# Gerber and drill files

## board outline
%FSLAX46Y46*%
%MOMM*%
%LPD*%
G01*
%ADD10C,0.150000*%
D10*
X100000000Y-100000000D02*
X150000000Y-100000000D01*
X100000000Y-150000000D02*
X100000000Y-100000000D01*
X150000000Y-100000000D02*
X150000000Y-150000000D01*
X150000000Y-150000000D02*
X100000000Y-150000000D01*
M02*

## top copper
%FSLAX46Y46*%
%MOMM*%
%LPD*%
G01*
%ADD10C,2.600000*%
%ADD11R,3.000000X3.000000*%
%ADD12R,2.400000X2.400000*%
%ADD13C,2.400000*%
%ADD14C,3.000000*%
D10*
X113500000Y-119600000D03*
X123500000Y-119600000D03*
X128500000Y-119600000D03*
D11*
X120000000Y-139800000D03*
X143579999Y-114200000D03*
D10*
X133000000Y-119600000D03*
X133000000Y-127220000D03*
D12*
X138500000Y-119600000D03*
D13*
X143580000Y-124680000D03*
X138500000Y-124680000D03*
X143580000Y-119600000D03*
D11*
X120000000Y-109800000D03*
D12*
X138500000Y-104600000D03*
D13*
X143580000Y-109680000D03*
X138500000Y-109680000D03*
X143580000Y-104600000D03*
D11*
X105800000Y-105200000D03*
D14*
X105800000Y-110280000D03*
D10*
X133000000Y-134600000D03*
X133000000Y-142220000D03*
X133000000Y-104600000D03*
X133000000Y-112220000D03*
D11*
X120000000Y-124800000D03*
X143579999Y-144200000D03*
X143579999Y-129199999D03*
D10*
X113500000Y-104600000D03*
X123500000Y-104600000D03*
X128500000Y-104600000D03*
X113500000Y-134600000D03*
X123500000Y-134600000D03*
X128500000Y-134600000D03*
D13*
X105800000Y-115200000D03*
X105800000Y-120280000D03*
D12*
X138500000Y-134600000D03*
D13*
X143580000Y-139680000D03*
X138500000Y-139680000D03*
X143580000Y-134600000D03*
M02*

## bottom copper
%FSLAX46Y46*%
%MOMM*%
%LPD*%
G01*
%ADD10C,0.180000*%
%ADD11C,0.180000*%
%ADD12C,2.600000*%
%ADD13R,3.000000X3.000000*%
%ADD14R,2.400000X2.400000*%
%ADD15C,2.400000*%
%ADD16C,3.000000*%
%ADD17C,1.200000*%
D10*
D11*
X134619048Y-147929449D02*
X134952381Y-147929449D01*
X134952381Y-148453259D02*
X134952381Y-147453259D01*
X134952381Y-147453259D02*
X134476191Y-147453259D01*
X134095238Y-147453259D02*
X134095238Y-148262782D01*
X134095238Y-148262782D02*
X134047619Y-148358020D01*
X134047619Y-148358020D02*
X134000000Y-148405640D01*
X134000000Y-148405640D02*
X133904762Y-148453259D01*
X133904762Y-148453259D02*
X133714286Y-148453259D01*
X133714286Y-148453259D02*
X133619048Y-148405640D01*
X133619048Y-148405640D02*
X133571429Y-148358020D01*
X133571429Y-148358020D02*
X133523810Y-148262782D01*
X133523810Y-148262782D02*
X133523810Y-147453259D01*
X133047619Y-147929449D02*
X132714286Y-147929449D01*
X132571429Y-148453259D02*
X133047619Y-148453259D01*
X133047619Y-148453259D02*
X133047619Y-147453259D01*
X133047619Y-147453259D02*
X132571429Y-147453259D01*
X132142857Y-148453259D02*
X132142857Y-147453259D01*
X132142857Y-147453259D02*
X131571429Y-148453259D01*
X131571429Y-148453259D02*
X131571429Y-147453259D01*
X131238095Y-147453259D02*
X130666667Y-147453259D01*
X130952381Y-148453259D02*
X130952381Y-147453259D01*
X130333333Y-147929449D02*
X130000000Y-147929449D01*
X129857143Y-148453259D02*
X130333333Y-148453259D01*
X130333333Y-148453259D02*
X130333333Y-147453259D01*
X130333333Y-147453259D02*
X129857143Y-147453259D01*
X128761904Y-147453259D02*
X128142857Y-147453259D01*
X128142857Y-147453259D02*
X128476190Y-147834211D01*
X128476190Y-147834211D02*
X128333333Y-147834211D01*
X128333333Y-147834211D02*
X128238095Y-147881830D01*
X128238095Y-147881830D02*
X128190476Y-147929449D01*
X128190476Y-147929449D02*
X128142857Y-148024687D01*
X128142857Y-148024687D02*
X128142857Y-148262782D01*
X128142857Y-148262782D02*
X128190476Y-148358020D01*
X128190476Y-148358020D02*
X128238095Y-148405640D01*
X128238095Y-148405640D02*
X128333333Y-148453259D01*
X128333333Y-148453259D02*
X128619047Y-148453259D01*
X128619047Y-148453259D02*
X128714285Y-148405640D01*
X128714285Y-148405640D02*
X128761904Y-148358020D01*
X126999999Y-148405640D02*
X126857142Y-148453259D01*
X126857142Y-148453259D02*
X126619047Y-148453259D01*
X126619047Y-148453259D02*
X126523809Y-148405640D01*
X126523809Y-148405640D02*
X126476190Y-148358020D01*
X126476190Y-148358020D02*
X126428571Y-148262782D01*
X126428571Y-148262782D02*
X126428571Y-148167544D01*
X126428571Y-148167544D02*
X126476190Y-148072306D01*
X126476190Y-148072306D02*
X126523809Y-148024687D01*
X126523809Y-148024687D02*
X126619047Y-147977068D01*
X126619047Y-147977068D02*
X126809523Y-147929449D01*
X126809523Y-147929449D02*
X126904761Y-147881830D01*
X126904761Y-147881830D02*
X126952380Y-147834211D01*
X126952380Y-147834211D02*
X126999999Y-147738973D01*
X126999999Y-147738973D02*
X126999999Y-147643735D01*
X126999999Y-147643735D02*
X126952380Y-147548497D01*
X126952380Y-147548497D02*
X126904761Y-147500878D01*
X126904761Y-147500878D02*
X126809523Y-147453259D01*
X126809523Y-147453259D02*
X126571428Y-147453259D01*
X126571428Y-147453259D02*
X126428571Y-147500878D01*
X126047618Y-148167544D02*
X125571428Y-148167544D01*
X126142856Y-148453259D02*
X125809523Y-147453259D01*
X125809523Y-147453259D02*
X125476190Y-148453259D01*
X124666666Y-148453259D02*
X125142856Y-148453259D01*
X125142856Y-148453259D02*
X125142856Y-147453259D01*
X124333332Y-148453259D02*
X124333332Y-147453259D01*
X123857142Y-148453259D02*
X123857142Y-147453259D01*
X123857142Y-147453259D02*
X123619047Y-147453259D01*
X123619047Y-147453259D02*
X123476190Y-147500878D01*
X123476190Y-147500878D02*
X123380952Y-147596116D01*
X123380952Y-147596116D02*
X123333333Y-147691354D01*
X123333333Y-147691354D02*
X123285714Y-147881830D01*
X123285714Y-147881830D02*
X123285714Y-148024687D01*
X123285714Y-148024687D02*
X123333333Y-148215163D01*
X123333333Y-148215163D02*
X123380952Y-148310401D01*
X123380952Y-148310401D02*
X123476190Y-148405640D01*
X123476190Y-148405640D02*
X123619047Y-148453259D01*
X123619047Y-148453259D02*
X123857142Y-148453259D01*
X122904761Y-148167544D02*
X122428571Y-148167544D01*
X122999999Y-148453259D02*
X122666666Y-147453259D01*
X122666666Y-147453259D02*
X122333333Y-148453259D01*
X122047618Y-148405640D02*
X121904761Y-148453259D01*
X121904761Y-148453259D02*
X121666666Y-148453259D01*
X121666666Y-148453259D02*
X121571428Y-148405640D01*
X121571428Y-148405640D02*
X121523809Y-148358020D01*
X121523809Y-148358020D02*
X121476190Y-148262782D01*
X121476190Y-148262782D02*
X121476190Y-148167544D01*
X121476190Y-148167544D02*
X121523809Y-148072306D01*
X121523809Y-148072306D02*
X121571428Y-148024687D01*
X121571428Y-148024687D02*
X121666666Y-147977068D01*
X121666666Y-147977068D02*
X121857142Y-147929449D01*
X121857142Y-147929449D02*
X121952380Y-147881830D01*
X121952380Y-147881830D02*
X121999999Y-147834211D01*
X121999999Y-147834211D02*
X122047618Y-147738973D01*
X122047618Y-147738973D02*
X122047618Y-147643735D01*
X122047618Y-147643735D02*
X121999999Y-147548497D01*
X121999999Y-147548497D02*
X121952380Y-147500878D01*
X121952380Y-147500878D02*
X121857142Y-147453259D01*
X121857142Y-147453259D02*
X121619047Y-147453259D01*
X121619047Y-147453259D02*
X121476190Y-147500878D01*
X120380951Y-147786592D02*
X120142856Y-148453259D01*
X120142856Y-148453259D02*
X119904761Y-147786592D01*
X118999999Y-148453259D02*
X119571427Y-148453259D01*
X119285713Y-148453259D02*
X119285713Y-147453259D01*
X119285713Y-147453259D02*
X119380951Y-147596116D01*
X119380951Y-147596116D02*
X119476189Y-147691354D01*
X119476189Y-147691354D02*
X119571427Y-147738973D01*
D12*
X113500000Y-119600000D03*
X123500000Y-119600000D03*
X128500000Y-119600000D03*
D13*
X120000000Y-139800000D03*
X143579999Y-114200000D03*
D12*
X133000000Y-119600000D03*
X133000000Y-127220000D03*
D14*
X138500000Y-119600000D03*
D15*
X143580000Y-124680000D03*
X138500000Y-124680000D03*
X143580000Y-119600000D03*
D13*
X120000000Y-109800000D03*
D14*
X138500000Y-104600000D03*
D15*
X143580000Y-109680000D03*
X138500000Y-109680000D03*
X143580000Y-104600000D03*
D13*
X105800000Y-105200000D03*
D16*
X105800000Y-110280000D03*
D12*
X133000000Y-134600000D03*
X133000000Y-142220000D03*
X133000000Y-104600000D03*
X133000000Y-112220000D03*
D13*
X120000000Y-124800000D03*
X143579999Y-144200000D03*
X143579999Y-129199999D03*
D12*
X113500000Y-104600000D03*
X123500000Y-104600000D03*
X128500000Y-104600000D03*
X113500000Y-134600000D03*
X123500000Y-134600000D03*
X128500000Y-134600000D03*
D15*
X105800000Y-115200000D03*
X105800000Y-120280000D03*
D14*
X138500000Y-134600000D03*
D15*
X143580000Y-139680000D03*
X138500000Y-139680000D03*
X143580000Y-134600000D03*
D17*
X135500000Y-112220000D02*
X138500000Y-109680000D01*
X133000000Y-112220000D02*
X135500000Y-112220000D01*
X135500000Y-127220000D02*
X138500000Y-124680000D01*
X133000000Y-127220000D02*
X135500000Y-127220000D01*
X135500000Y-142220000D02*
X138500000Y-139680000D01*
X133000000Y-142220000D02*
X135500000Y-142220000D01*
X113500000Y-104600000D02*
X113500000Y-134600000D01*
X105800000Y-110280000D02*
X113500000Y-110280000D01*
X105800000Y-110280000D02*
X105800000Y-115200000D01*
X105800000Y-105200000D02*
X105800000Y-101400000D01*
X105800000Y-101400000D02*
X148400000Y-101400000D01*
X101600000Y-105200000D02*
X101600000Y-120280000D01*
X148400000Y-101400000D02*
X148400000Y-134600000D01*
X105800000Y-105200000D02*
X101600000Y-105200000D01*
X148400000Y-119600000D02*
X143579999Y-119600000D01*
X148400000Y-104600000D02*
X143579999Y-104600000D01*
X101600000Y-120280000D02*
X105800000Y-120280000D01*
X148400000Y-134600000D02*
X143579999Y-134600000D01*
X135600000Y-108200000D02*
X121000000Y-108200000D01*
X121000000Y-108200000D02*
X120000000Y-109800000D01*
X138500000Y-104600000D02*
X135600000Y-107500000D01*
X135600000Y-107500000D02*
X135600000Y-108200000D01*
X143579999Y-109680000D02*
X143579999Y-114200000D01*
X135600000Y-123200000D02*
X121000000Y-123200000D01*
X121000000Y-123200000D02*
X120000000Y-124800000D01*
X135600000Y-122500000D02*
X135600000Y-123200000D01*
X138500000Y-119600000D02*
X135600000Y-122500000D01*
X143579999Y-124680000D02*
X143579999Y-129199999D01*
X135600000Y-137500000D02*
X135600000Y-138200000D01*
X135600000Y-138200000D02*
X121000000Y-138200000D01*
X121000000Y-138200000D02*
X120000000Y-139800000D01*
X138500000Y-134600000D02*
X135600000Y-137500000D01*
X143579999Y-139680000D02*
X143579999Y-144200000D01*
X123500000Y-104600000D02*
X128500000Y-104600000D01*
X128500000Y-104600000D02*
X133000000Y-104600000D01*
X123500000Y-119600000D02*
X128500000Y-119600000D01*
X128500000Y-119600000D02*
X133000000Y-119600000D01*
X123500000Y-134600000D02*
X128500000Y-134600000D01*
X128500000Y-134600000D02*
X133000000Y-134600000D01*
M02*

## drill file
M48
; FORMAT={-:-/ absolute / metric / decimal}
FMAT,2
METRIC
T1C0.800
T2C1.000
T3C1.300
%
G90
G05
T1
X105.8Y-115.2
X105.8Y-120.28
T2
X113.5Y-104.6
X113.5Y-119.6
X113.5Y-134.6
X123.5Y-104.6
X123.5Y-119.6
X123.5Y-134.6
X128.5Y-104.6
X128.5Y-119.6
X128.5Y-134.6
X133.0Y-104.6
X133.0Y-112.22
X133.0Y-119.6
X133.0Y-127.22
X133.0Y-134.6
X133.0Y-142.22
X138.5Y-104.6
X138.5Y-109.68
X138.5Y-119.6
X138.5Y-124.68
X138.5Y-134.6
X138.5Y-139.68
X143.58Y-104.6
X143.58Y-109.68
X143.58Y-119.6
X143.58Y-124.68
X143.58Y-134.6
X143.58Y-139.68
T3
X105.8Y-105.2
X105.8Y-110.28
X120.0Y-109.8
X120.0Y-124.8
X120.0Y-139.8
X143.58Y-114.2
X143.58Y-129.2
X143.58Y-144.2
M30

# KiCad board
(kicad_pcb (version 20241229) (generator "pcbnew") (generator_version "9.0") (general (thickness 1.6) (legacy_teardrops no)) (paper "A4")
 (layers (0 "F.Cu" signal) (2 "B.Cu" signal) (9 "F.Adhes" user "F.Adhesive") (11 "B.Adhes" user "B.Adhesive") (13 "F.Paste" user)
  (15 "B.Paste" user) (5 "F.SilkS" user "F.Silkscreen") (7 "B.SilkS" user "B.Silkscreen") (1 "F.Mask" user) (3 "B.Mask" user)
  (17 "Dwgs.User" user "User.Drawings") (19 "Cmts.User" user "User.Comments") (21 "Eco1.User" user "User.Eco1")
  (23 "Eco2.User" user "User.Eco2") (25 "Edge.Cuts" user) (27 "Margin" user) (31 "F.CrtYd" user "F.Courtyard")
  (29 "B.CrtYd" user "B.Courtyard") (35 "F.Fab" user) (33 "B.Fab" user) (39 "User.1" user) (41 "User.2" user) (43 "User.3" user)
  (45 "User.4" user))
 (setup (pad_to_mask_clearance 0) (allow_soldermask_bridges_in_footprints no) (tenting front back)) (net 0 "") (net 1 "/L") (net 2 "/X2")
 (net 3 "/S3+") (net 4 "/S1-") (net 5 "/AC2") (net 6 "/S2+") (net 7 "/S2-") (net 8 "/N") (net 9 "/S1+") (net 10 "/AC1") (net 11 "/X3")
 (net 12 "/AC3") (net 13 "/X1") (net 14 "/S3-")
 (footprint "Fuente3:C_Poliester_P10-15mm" (layer "F.Cu") (at 113.5 119.6)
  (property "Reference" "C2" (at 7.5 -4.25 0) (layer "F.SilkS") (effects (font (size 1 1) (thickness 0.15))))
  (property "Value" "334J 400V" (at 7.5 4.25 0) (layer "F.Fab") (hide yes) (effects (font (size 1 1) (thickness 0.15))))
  (pad "1" thru_hole circle (at 0 0) (size 2.6 2.6) (drill 1) (layers "B.Cu" "B.Mask") (remove_unused_layers no) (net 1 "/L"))
  (pad "2" thru_hole circle (at 10 0) (size 2.6 2.6) (drill 1) (layers "B.Cu" "B.Mask") (remove_unused_layers no) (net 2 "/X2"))
  (pad "2" thru_hole circle (at 15 0) (size 2.6 2.6) (drill 1) (layers "B.Cu" "B.Mask") (remove_unused_layers no) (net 2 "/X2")))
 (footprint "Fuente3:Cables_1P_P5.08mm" (layer "F.Cu") (at 120 139.8)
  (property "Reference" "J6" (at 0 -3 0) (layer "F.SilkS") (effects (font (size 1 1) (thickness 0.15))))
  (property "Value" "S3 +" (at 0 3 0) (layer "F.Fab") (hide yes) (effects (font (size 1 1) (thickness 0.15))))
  (pad "1" thru_hole rect (at 0 0) (size 3 3) (drill 1.3) (layers "B.Cu" "B.Mask") (remove_unused_layers no) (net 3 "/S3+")))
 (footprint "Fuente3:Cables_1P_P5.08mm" (layer "F.Cu") (at 143.579999 114.2)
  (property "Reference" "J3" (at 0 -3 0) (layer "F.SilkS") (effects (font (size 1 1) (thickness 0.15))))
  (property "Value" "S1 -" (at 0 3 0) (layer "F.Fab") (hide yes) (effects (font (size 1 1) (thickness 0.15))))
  (pad "1" thru_hole rect (at 0 0) (size 3 3) (drill 1.3) (layers "B.Cu" "B.Mask") (remove_unused_layers no) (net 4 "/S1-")))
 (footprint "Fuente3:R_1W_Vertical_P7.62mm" (layer "F.Cu") (at 133 119.6 -90)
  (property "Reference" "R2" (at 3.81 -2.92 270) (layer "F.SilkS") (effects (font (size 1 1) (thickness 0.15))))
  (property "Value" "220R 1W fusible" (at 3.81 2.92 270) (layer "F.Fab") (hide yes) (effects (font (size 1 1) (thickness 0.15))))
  (pad "1" thru_hole circle (at 0 0 270) (size 2.6 2.6) (drill 1) (layers "B.Cu" "B.Mask") (remove_unused_layers no) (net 2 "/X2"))
  (pad "2" thru_hole circle (at 7.62 0 270) (size 2.6 2.6) (drill 1) (layers "B.Cu" "B.Mask") (remove_unused_layers no) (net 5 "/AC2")))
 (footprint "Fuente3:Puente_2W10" (layer "F.Cu") (at 138.5 119.6)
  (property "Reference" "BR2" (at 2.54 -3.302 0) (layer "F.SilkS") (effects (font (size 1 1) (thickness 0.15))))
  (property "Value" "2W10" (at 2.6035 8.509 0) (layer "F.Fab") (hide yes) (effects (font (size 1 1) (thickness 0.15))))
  (pad "1" thru_hole rect (at 0 0) (size 2.4 2.4) (drill 1) (layers "B.Cu" "B.Mask") (remove_unused_layers no) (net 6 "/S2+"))
  (pad "2" thru_hole circle (at 5.08 5.08) (size 2.4 2.4) (drill 1) (layers "B.Cu" "B.Mask") (remove_unused_layers no) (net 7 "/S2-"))
  (pad "3" thru_hole circle (at 0 5.08) (size 2.4 2.4) (drill 1) (layers "B.Cu" "B.Mask") (remove_unused_layers no) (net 5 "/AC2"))
  (pad "4" thru_hole circle (at 5.08 0) (size 2.4 2.4) (drill 1) (layers "B.Cu" "B.Mask") (remove_unused_layers no) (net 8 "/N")))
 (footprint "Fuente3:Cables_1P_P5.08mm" (layer "F.Cu") (at 120 109.8)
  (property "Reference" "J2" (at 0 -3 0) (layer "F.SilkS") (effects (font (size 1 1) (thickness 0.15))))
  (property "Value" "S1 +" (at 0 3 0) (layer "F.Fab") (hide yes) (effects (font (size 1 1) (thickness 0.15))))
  (pad "1" thru_hole rect (at 0 0) (size 3 3) (drill 1.3) (layers "B.Cu" "B.Mask") (remove_unused_layers no) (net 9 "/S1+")))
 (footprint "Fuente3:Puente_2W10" (layer "F.Cu") (at 138.5 104.6)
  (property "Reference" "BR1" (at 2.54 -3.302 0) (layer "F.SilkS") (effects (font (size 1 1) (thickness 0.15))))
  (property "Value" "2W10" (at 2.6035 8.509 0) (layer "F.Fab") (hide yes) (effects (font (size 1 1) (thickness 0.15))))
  (pad "1" thru_hole rect (at 0 0) (size 2.4 2.4) (drill 1) (layers "B.Cu" "B.Mask") (remove_unused_layers no) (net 9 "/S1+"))
  (pad "2" thru_hole circle (at 5.08 5.08) (size 2.4 2.4) (drill 1) (layers "B.Cu" "B.Mask") (remove_unused_layers no) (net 4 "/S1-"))
  (pad "3" thru_hole circle (at 0 5.08) (size 2.4 2.4) (drill 1) (layers "B.Cu" "B.Mask") (remove_unused_layers no) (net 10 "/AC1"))
  (pad "4" thru_hole circle (at 5.08 0) (size 2.4 2.4) (drill 1) (layers "B.Cu" "B.Mask") (remove_unused_layers no) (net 8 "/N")))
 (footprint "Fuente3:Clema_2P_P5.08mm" (layer "F.Cu") (at 105.8 105.2 -90)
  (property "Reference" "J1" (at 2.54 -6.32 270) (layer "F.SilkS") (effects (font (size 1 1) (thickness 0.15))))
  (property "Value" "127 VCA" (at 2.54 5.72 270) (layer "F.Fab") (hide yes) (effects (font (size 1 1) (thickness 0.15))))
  (pad "1" thru_hole rect (at 0 0 270) (size 3 3) (drill 1.3) (layers "B.Cu" "B.Mask") (remove_unused_layers no) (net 8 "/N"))
  (pad "2" thru_hole circle (at 5.08 0 270) (size 3 3) (drill 1.3) (layers "B.Cu" "B.Mask") (remove_unused_layers no) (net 1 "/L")))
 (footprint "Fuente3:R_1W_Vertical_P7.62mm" (layer "F.Cu") (at 133 134.6 -90)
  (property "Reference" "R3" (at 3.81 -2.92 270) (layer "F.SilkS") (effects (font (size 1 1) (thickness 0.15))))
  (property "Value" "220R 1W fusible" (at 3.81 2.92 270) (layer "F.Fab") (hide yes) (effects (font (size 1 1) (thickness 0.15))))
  (pad "1" thru_hole circle (at 0 0 270) (size 2.6 2.6) (drill 1) (layers "B.Cu" "B.Mask") (remove_unused_layers no) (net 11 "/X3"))
  (pad "2" thru_hole circle (at 7.62 0 270) (size 2.6 2.6) (drill 1) (layers "B.Cu" "B.Mask") (remove_unused_layers no) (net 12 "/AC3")))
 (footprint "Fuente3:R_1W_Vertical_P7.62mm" (layer "F.Cu") (at 133 104.6 -90)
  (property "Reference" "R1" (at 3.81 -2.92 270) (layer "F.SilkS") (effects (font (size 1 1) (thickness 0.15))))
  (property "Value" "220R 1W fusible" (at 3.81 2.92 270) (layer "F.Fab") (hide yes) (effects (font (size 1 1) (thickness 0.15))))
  (pad "1" thru_hole circle (at 0 0 270) (size 2.6 2.6) (drill 1) (layers "B.Cu" "B.Mask") (remove_unused_layers no) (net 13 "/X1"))
  (pad "2" thru_hole circle (at 7.62 0 270) (size 2.6 2.6) (drill 1) (layers "B.Cu" "B.Mask") (remove_unused_layers no) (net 10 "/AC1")))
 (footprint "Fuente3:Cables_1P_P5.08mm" (layer "F.Cu") (at 120 124.8)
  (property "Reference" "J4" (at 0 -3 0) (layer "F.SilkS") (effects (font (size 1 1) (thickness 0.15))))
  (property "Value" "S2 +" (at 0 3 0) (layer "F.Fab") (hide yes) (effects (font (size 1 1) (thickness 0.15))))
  (pad "1" thru_hole rect (at 0 0) (size 3 3) (drill 1.3) (layers "B.Cu" "B.Mask") (remove_unused_layers no) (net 6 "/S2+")))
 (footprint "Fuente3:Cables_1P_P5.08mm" (layer "F.Cu") (at 143.579999 144.2)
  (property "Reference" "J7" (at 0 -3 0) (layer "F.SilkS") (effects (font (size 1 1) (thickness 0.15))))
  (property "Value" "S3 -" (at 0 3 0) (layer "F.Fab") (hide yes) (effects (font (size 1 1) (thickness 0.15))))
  (pad "1" thru_hole rect (at 0 0) (size 3 3) (drill 1.3) (layers "B.Cu" "B.Mask") (remove_unused_layers no) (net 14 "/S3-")))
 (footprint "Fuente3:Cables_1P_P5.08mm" (layer "F.Cu") (at 143.579999 129.199999)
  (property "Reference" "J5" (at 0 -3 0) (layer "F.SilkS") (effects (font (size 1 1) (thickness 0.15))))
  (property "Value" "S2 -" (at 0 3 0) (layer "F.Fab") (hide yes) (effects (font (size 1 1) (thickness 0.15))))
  (pad "1" thru_hole rect (at 0 0) (size 3 3) (drill 1.3) (layers "B.Cu" "B.Mask") (remove_unused_layers no) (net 7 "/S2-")))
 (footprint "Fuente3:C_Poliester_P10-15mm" (layer "F.Cu") (at 113.5 104.6)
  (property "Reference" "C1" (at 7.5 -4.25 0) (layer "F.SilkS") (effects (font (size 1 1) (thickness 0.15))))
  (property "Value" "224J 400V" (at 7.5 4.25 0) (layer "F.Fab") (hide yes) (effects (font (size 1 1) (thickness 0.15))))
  (pad "1" thru_hole circle (at 0 0) (size 2.6 2.6) (drill 1) (layers "B.Cu" "B.Mask") (remove_unused_layers no) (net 1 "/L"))
  (pad "2" thru_hole circle (at 10 0) (size 2.6 2.6) (drill 1) (layers "B.Cu" "B.Mask") (remove_unused_layers no) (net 13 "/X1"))
  (pad "2" thru_hole circle (at 15 0) (size 2.6 2.6) (drill 1) (layers "B.Cu" "B.Mask") (remove_unused_layers no) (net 13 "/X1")))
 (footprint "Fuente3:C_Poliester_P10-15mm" (layer "F.Cu") (at 113.5 134.6)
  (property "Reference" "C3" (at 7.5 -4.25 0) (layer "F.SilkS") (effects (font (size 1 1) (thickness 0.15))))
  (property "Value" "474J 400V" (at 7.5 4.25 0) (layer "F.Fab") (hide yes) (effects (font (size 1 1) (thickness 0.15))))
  (pad "1" thru_hole circle (at 0 0) (size 2.6 2.6) (drill 1) (layers "B.Cu" "B.Mask") (remove_unused_layers no) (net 1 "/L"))
  (pad "2" thru_hole circle (at 10 0) (size 2.6 2.6) (drill 1) (layers "B.Cu" "B.Mask") (remove_unused_layers no) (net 11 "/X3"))
  (pad "2" thru_hole circle (at 15 0) (size 2.6 2.6) (drill 1) (layers "B.Cu" "B.Mask") (remove_unused_layers no) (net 11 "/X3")))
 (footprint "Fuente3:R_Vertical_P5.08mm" (layer "F.Cu") (at 105.8 115.2 -90)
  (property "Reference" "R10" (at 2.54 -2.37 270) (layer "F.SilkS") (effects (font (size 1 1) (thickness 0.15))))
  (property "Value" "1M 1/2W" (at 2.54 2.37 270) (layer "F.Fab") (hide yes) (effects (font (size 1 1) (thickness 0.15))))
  (pad "1" thru_hole circle (at 0 0 270) (size 2.4 2.4) (drill 0.8) (layers "B.Cu" "B.Mask") (remove_unused_layers no) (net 1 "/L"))
  (pad "2" thru_hole circle (at 5.08 0 270) (size 2.4 2.4) (drill 0.8) (layers "B.Cu" "B.Mask") (remove_unused_layers no) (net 8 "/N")))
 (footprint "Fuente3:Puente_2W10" (layer "F.Cu") (at 138.5 134.6)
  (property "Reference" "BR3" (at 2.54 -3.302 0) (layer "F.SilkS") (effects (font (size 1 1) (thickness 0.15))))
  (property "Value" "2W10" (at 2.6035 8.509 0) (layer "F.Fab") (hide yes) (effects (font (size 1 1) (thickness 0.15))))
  (pad "1" thru_hole rect (at 0 0) (size 2.4 2.4) (drill 1) (layers "B.Cu" "B.Mask") (remove_unused_layers no) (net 3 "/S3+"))
  (pad "2" thru_hole circle (at 5.08 5.08) (size 2.4 2.4) (drill 1) (layers "B.Cu" "B.Mask") (remove_unused_layers no) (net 14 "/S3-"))
  (pad "3" thru_hole circle (at 0 5.08) (size 2.4 2.4) (drill 1) (layers "B.Cu" "B.Mask") (remove_unused_layers no) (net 12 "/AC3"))
  (pad "4" thru_hole circle (at 5.08 0) (size 2.4 2.4) (drill 1) (layers "B.Cu" "B.Mask") (remove_unused_layers no) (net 8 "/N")))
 (gr_line (start 100 100) (end 150 100) (stroke (width 0.15) (type default)) (layer "Edge.Cuts"))
 (gr_line (start 100 150) (end 100 100) (stroke (width 0.15) (type default)) (layer "Edge.Cuts"))
 (gr_line (start 150 100) (end 150 150) (stroke (width 0.15) (type default)) (layer "Edge.Cuts"))
 (gr_line (start 150 150) (end 100 150) (stroke (width 0.15) (type default)) (layer "Edge.Cuts"))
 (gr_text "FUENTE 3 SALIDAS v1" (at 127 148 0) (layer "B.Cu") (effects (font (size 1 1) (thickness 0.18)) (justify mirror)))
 (segment (start 135.5 112.22) (end 138.5 109.68) (width 1.2) (layer "B.Cu") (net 10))
 (segment (start 133 112.22) (end 135.5 112.22) (width 1.2) (layer "B.Cu") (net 10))
 (segment (start 135.5 127.22) (end 138.5 124.68) (width 1.2) (layer "B.Cu") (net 5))
 (segment (start 133 127.22) (end 135.5 127.22) (width 1.2) (layer "B.Cu") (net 5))
 (segment (start 135.5 142.22) (end 138.5 139.68) (width 1.2) (layer "B.Cu") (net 12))
 (segment (start 133 142.22) (end 135.5 142.22) (width 1.2) (layer "B.Cu") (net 12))
 (segment (start 113.5 104.6) (end 113.5 134.6) (width 1.2) (layer "B.Cu") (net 1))
 (segment (start 105.8 110.28) (end 113.5 110.28) (width 1.2) (layer "B.Cu") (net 1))
 (segment (start 105.8 110.28) (end 105.8 115.2) (width 1.2) (layer "B.Cu") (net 1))
 (segment (start 105.8 105.2) (end 105.8 101.4) (width 1.2) (layer "B.Cu") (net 8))
 (segment (start 105.8 101.4) (end 148.4 101.4) (width 1.2) (layer "B.Cu") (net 8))
 (segment (start 101.6 105.2) (end 101.6 120.28) (width 1.2) (layer "B.Cu") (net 8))
 (segment (start 148.4 101.4) (end 148.4 134.6) (width 1.2) (layer "B.Cu") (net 8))
 (segment (start 105.8 105.2) (end 101.6 105.2) (width 1.2) (layer "B.Cu") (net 8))
 (segment (start 148.4 119.6) (end 143.579999 119.6) (width 1.2) (layer "B.Cu") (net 8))
 (segment (start 148.4 104.6) (end 143.579999 104.6) (width 1.2) (layer "B.Cu") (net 8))
 (segment (start 101.6 120.28) (end 105.8 120.28) (width 1.2) (layer "B.Cu") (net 8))
 (segment (start 148.4 134.6) (end 143.579999 134.6) (width 1.2) (layer "B.Cu") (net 8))
 (segment (start 135.6 108.2) (end 121 108.2) (width 1.2) (layer "B.Cu") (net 9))
 (segment (start 121 108.2) (end 120 109.8) (width 1.2) (layer "B.Cu") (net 9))
 (segment (start 138.5 104.6) (end 135.6 107.5) (width 1.2) (layer "B.Cu") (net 9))
 (segment (start 135.6 107.5) (end 135.6 108.2) (width 1.2) (layer "B.Cu") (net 9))
 (segment (start 143.579999 109.68) (end 143.579999 114.2) (width 1.2) (layer "B.Cu") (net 4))
 (segment (start 135.6 123.2) (end 121 123.2) (width 1.2) (layer "B.Cu") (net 6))
 (segment (start 121 123.2) (end 120 124.8) (width 1.2) (layer "B.Cu") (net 6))
 (segment (start 135.6 122.5) (end 135.6 123.2) (width 1.2) (layer "B.Cu") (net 6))
 (segment (start 138.5 119.6) (end 135.6 122.5) (width 1.2) (layer "B.Cu") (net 6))
 (segment (start 143.579999 124.68) (end 143.579999 129.199999) (width 1.2) (layer "B.Cu") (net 7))
 (segment (start 135.6 137.5) (end 135.6 138.2) (width 1.2) (layer "B.Cu") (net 3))
 (segment (start 135.6 138.2) (end 121 138.2) (width 1.2) (layer "B.Cu") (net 3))
 (segment (start 121 138.2) (end 120 139.8) (width 1.2) (layer "B.Cu") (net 3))
 (segment (start 138.5 134.6) (end 135.6 137.5) (width 1.2) (layer "B.Cu") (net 3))
 (segment (start 143.579999 139.68) (end 143.579999 144.2) (width 1.2) (layer "B.Cu") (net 14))
 (segment (start 123.5 104.6) (end 128.5 104.6) (width 1.2) (layer "B.Cu") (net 13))
 (segment (start 128.5 104.6) (end 133 104.6) (width 1.2) (layer "B.Cu") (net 13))
 (segment (start 123.5 119.6) (end 128.5 119.6) (width 1.2) (layer "B.Cu") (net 2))
 (segment (start 128.5 119.6) (end 133 119.6) (width 1.2) (layer "B.Cu") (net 2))
 (segment (start 123.5 134.6) (end 128.5 134.6) (width 1.2) (layer "B.Cu") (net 11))
 (segment (start 128.5 134.6) (end 133 134.6) (width 1.2) (layer "B.Cu") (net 11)))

